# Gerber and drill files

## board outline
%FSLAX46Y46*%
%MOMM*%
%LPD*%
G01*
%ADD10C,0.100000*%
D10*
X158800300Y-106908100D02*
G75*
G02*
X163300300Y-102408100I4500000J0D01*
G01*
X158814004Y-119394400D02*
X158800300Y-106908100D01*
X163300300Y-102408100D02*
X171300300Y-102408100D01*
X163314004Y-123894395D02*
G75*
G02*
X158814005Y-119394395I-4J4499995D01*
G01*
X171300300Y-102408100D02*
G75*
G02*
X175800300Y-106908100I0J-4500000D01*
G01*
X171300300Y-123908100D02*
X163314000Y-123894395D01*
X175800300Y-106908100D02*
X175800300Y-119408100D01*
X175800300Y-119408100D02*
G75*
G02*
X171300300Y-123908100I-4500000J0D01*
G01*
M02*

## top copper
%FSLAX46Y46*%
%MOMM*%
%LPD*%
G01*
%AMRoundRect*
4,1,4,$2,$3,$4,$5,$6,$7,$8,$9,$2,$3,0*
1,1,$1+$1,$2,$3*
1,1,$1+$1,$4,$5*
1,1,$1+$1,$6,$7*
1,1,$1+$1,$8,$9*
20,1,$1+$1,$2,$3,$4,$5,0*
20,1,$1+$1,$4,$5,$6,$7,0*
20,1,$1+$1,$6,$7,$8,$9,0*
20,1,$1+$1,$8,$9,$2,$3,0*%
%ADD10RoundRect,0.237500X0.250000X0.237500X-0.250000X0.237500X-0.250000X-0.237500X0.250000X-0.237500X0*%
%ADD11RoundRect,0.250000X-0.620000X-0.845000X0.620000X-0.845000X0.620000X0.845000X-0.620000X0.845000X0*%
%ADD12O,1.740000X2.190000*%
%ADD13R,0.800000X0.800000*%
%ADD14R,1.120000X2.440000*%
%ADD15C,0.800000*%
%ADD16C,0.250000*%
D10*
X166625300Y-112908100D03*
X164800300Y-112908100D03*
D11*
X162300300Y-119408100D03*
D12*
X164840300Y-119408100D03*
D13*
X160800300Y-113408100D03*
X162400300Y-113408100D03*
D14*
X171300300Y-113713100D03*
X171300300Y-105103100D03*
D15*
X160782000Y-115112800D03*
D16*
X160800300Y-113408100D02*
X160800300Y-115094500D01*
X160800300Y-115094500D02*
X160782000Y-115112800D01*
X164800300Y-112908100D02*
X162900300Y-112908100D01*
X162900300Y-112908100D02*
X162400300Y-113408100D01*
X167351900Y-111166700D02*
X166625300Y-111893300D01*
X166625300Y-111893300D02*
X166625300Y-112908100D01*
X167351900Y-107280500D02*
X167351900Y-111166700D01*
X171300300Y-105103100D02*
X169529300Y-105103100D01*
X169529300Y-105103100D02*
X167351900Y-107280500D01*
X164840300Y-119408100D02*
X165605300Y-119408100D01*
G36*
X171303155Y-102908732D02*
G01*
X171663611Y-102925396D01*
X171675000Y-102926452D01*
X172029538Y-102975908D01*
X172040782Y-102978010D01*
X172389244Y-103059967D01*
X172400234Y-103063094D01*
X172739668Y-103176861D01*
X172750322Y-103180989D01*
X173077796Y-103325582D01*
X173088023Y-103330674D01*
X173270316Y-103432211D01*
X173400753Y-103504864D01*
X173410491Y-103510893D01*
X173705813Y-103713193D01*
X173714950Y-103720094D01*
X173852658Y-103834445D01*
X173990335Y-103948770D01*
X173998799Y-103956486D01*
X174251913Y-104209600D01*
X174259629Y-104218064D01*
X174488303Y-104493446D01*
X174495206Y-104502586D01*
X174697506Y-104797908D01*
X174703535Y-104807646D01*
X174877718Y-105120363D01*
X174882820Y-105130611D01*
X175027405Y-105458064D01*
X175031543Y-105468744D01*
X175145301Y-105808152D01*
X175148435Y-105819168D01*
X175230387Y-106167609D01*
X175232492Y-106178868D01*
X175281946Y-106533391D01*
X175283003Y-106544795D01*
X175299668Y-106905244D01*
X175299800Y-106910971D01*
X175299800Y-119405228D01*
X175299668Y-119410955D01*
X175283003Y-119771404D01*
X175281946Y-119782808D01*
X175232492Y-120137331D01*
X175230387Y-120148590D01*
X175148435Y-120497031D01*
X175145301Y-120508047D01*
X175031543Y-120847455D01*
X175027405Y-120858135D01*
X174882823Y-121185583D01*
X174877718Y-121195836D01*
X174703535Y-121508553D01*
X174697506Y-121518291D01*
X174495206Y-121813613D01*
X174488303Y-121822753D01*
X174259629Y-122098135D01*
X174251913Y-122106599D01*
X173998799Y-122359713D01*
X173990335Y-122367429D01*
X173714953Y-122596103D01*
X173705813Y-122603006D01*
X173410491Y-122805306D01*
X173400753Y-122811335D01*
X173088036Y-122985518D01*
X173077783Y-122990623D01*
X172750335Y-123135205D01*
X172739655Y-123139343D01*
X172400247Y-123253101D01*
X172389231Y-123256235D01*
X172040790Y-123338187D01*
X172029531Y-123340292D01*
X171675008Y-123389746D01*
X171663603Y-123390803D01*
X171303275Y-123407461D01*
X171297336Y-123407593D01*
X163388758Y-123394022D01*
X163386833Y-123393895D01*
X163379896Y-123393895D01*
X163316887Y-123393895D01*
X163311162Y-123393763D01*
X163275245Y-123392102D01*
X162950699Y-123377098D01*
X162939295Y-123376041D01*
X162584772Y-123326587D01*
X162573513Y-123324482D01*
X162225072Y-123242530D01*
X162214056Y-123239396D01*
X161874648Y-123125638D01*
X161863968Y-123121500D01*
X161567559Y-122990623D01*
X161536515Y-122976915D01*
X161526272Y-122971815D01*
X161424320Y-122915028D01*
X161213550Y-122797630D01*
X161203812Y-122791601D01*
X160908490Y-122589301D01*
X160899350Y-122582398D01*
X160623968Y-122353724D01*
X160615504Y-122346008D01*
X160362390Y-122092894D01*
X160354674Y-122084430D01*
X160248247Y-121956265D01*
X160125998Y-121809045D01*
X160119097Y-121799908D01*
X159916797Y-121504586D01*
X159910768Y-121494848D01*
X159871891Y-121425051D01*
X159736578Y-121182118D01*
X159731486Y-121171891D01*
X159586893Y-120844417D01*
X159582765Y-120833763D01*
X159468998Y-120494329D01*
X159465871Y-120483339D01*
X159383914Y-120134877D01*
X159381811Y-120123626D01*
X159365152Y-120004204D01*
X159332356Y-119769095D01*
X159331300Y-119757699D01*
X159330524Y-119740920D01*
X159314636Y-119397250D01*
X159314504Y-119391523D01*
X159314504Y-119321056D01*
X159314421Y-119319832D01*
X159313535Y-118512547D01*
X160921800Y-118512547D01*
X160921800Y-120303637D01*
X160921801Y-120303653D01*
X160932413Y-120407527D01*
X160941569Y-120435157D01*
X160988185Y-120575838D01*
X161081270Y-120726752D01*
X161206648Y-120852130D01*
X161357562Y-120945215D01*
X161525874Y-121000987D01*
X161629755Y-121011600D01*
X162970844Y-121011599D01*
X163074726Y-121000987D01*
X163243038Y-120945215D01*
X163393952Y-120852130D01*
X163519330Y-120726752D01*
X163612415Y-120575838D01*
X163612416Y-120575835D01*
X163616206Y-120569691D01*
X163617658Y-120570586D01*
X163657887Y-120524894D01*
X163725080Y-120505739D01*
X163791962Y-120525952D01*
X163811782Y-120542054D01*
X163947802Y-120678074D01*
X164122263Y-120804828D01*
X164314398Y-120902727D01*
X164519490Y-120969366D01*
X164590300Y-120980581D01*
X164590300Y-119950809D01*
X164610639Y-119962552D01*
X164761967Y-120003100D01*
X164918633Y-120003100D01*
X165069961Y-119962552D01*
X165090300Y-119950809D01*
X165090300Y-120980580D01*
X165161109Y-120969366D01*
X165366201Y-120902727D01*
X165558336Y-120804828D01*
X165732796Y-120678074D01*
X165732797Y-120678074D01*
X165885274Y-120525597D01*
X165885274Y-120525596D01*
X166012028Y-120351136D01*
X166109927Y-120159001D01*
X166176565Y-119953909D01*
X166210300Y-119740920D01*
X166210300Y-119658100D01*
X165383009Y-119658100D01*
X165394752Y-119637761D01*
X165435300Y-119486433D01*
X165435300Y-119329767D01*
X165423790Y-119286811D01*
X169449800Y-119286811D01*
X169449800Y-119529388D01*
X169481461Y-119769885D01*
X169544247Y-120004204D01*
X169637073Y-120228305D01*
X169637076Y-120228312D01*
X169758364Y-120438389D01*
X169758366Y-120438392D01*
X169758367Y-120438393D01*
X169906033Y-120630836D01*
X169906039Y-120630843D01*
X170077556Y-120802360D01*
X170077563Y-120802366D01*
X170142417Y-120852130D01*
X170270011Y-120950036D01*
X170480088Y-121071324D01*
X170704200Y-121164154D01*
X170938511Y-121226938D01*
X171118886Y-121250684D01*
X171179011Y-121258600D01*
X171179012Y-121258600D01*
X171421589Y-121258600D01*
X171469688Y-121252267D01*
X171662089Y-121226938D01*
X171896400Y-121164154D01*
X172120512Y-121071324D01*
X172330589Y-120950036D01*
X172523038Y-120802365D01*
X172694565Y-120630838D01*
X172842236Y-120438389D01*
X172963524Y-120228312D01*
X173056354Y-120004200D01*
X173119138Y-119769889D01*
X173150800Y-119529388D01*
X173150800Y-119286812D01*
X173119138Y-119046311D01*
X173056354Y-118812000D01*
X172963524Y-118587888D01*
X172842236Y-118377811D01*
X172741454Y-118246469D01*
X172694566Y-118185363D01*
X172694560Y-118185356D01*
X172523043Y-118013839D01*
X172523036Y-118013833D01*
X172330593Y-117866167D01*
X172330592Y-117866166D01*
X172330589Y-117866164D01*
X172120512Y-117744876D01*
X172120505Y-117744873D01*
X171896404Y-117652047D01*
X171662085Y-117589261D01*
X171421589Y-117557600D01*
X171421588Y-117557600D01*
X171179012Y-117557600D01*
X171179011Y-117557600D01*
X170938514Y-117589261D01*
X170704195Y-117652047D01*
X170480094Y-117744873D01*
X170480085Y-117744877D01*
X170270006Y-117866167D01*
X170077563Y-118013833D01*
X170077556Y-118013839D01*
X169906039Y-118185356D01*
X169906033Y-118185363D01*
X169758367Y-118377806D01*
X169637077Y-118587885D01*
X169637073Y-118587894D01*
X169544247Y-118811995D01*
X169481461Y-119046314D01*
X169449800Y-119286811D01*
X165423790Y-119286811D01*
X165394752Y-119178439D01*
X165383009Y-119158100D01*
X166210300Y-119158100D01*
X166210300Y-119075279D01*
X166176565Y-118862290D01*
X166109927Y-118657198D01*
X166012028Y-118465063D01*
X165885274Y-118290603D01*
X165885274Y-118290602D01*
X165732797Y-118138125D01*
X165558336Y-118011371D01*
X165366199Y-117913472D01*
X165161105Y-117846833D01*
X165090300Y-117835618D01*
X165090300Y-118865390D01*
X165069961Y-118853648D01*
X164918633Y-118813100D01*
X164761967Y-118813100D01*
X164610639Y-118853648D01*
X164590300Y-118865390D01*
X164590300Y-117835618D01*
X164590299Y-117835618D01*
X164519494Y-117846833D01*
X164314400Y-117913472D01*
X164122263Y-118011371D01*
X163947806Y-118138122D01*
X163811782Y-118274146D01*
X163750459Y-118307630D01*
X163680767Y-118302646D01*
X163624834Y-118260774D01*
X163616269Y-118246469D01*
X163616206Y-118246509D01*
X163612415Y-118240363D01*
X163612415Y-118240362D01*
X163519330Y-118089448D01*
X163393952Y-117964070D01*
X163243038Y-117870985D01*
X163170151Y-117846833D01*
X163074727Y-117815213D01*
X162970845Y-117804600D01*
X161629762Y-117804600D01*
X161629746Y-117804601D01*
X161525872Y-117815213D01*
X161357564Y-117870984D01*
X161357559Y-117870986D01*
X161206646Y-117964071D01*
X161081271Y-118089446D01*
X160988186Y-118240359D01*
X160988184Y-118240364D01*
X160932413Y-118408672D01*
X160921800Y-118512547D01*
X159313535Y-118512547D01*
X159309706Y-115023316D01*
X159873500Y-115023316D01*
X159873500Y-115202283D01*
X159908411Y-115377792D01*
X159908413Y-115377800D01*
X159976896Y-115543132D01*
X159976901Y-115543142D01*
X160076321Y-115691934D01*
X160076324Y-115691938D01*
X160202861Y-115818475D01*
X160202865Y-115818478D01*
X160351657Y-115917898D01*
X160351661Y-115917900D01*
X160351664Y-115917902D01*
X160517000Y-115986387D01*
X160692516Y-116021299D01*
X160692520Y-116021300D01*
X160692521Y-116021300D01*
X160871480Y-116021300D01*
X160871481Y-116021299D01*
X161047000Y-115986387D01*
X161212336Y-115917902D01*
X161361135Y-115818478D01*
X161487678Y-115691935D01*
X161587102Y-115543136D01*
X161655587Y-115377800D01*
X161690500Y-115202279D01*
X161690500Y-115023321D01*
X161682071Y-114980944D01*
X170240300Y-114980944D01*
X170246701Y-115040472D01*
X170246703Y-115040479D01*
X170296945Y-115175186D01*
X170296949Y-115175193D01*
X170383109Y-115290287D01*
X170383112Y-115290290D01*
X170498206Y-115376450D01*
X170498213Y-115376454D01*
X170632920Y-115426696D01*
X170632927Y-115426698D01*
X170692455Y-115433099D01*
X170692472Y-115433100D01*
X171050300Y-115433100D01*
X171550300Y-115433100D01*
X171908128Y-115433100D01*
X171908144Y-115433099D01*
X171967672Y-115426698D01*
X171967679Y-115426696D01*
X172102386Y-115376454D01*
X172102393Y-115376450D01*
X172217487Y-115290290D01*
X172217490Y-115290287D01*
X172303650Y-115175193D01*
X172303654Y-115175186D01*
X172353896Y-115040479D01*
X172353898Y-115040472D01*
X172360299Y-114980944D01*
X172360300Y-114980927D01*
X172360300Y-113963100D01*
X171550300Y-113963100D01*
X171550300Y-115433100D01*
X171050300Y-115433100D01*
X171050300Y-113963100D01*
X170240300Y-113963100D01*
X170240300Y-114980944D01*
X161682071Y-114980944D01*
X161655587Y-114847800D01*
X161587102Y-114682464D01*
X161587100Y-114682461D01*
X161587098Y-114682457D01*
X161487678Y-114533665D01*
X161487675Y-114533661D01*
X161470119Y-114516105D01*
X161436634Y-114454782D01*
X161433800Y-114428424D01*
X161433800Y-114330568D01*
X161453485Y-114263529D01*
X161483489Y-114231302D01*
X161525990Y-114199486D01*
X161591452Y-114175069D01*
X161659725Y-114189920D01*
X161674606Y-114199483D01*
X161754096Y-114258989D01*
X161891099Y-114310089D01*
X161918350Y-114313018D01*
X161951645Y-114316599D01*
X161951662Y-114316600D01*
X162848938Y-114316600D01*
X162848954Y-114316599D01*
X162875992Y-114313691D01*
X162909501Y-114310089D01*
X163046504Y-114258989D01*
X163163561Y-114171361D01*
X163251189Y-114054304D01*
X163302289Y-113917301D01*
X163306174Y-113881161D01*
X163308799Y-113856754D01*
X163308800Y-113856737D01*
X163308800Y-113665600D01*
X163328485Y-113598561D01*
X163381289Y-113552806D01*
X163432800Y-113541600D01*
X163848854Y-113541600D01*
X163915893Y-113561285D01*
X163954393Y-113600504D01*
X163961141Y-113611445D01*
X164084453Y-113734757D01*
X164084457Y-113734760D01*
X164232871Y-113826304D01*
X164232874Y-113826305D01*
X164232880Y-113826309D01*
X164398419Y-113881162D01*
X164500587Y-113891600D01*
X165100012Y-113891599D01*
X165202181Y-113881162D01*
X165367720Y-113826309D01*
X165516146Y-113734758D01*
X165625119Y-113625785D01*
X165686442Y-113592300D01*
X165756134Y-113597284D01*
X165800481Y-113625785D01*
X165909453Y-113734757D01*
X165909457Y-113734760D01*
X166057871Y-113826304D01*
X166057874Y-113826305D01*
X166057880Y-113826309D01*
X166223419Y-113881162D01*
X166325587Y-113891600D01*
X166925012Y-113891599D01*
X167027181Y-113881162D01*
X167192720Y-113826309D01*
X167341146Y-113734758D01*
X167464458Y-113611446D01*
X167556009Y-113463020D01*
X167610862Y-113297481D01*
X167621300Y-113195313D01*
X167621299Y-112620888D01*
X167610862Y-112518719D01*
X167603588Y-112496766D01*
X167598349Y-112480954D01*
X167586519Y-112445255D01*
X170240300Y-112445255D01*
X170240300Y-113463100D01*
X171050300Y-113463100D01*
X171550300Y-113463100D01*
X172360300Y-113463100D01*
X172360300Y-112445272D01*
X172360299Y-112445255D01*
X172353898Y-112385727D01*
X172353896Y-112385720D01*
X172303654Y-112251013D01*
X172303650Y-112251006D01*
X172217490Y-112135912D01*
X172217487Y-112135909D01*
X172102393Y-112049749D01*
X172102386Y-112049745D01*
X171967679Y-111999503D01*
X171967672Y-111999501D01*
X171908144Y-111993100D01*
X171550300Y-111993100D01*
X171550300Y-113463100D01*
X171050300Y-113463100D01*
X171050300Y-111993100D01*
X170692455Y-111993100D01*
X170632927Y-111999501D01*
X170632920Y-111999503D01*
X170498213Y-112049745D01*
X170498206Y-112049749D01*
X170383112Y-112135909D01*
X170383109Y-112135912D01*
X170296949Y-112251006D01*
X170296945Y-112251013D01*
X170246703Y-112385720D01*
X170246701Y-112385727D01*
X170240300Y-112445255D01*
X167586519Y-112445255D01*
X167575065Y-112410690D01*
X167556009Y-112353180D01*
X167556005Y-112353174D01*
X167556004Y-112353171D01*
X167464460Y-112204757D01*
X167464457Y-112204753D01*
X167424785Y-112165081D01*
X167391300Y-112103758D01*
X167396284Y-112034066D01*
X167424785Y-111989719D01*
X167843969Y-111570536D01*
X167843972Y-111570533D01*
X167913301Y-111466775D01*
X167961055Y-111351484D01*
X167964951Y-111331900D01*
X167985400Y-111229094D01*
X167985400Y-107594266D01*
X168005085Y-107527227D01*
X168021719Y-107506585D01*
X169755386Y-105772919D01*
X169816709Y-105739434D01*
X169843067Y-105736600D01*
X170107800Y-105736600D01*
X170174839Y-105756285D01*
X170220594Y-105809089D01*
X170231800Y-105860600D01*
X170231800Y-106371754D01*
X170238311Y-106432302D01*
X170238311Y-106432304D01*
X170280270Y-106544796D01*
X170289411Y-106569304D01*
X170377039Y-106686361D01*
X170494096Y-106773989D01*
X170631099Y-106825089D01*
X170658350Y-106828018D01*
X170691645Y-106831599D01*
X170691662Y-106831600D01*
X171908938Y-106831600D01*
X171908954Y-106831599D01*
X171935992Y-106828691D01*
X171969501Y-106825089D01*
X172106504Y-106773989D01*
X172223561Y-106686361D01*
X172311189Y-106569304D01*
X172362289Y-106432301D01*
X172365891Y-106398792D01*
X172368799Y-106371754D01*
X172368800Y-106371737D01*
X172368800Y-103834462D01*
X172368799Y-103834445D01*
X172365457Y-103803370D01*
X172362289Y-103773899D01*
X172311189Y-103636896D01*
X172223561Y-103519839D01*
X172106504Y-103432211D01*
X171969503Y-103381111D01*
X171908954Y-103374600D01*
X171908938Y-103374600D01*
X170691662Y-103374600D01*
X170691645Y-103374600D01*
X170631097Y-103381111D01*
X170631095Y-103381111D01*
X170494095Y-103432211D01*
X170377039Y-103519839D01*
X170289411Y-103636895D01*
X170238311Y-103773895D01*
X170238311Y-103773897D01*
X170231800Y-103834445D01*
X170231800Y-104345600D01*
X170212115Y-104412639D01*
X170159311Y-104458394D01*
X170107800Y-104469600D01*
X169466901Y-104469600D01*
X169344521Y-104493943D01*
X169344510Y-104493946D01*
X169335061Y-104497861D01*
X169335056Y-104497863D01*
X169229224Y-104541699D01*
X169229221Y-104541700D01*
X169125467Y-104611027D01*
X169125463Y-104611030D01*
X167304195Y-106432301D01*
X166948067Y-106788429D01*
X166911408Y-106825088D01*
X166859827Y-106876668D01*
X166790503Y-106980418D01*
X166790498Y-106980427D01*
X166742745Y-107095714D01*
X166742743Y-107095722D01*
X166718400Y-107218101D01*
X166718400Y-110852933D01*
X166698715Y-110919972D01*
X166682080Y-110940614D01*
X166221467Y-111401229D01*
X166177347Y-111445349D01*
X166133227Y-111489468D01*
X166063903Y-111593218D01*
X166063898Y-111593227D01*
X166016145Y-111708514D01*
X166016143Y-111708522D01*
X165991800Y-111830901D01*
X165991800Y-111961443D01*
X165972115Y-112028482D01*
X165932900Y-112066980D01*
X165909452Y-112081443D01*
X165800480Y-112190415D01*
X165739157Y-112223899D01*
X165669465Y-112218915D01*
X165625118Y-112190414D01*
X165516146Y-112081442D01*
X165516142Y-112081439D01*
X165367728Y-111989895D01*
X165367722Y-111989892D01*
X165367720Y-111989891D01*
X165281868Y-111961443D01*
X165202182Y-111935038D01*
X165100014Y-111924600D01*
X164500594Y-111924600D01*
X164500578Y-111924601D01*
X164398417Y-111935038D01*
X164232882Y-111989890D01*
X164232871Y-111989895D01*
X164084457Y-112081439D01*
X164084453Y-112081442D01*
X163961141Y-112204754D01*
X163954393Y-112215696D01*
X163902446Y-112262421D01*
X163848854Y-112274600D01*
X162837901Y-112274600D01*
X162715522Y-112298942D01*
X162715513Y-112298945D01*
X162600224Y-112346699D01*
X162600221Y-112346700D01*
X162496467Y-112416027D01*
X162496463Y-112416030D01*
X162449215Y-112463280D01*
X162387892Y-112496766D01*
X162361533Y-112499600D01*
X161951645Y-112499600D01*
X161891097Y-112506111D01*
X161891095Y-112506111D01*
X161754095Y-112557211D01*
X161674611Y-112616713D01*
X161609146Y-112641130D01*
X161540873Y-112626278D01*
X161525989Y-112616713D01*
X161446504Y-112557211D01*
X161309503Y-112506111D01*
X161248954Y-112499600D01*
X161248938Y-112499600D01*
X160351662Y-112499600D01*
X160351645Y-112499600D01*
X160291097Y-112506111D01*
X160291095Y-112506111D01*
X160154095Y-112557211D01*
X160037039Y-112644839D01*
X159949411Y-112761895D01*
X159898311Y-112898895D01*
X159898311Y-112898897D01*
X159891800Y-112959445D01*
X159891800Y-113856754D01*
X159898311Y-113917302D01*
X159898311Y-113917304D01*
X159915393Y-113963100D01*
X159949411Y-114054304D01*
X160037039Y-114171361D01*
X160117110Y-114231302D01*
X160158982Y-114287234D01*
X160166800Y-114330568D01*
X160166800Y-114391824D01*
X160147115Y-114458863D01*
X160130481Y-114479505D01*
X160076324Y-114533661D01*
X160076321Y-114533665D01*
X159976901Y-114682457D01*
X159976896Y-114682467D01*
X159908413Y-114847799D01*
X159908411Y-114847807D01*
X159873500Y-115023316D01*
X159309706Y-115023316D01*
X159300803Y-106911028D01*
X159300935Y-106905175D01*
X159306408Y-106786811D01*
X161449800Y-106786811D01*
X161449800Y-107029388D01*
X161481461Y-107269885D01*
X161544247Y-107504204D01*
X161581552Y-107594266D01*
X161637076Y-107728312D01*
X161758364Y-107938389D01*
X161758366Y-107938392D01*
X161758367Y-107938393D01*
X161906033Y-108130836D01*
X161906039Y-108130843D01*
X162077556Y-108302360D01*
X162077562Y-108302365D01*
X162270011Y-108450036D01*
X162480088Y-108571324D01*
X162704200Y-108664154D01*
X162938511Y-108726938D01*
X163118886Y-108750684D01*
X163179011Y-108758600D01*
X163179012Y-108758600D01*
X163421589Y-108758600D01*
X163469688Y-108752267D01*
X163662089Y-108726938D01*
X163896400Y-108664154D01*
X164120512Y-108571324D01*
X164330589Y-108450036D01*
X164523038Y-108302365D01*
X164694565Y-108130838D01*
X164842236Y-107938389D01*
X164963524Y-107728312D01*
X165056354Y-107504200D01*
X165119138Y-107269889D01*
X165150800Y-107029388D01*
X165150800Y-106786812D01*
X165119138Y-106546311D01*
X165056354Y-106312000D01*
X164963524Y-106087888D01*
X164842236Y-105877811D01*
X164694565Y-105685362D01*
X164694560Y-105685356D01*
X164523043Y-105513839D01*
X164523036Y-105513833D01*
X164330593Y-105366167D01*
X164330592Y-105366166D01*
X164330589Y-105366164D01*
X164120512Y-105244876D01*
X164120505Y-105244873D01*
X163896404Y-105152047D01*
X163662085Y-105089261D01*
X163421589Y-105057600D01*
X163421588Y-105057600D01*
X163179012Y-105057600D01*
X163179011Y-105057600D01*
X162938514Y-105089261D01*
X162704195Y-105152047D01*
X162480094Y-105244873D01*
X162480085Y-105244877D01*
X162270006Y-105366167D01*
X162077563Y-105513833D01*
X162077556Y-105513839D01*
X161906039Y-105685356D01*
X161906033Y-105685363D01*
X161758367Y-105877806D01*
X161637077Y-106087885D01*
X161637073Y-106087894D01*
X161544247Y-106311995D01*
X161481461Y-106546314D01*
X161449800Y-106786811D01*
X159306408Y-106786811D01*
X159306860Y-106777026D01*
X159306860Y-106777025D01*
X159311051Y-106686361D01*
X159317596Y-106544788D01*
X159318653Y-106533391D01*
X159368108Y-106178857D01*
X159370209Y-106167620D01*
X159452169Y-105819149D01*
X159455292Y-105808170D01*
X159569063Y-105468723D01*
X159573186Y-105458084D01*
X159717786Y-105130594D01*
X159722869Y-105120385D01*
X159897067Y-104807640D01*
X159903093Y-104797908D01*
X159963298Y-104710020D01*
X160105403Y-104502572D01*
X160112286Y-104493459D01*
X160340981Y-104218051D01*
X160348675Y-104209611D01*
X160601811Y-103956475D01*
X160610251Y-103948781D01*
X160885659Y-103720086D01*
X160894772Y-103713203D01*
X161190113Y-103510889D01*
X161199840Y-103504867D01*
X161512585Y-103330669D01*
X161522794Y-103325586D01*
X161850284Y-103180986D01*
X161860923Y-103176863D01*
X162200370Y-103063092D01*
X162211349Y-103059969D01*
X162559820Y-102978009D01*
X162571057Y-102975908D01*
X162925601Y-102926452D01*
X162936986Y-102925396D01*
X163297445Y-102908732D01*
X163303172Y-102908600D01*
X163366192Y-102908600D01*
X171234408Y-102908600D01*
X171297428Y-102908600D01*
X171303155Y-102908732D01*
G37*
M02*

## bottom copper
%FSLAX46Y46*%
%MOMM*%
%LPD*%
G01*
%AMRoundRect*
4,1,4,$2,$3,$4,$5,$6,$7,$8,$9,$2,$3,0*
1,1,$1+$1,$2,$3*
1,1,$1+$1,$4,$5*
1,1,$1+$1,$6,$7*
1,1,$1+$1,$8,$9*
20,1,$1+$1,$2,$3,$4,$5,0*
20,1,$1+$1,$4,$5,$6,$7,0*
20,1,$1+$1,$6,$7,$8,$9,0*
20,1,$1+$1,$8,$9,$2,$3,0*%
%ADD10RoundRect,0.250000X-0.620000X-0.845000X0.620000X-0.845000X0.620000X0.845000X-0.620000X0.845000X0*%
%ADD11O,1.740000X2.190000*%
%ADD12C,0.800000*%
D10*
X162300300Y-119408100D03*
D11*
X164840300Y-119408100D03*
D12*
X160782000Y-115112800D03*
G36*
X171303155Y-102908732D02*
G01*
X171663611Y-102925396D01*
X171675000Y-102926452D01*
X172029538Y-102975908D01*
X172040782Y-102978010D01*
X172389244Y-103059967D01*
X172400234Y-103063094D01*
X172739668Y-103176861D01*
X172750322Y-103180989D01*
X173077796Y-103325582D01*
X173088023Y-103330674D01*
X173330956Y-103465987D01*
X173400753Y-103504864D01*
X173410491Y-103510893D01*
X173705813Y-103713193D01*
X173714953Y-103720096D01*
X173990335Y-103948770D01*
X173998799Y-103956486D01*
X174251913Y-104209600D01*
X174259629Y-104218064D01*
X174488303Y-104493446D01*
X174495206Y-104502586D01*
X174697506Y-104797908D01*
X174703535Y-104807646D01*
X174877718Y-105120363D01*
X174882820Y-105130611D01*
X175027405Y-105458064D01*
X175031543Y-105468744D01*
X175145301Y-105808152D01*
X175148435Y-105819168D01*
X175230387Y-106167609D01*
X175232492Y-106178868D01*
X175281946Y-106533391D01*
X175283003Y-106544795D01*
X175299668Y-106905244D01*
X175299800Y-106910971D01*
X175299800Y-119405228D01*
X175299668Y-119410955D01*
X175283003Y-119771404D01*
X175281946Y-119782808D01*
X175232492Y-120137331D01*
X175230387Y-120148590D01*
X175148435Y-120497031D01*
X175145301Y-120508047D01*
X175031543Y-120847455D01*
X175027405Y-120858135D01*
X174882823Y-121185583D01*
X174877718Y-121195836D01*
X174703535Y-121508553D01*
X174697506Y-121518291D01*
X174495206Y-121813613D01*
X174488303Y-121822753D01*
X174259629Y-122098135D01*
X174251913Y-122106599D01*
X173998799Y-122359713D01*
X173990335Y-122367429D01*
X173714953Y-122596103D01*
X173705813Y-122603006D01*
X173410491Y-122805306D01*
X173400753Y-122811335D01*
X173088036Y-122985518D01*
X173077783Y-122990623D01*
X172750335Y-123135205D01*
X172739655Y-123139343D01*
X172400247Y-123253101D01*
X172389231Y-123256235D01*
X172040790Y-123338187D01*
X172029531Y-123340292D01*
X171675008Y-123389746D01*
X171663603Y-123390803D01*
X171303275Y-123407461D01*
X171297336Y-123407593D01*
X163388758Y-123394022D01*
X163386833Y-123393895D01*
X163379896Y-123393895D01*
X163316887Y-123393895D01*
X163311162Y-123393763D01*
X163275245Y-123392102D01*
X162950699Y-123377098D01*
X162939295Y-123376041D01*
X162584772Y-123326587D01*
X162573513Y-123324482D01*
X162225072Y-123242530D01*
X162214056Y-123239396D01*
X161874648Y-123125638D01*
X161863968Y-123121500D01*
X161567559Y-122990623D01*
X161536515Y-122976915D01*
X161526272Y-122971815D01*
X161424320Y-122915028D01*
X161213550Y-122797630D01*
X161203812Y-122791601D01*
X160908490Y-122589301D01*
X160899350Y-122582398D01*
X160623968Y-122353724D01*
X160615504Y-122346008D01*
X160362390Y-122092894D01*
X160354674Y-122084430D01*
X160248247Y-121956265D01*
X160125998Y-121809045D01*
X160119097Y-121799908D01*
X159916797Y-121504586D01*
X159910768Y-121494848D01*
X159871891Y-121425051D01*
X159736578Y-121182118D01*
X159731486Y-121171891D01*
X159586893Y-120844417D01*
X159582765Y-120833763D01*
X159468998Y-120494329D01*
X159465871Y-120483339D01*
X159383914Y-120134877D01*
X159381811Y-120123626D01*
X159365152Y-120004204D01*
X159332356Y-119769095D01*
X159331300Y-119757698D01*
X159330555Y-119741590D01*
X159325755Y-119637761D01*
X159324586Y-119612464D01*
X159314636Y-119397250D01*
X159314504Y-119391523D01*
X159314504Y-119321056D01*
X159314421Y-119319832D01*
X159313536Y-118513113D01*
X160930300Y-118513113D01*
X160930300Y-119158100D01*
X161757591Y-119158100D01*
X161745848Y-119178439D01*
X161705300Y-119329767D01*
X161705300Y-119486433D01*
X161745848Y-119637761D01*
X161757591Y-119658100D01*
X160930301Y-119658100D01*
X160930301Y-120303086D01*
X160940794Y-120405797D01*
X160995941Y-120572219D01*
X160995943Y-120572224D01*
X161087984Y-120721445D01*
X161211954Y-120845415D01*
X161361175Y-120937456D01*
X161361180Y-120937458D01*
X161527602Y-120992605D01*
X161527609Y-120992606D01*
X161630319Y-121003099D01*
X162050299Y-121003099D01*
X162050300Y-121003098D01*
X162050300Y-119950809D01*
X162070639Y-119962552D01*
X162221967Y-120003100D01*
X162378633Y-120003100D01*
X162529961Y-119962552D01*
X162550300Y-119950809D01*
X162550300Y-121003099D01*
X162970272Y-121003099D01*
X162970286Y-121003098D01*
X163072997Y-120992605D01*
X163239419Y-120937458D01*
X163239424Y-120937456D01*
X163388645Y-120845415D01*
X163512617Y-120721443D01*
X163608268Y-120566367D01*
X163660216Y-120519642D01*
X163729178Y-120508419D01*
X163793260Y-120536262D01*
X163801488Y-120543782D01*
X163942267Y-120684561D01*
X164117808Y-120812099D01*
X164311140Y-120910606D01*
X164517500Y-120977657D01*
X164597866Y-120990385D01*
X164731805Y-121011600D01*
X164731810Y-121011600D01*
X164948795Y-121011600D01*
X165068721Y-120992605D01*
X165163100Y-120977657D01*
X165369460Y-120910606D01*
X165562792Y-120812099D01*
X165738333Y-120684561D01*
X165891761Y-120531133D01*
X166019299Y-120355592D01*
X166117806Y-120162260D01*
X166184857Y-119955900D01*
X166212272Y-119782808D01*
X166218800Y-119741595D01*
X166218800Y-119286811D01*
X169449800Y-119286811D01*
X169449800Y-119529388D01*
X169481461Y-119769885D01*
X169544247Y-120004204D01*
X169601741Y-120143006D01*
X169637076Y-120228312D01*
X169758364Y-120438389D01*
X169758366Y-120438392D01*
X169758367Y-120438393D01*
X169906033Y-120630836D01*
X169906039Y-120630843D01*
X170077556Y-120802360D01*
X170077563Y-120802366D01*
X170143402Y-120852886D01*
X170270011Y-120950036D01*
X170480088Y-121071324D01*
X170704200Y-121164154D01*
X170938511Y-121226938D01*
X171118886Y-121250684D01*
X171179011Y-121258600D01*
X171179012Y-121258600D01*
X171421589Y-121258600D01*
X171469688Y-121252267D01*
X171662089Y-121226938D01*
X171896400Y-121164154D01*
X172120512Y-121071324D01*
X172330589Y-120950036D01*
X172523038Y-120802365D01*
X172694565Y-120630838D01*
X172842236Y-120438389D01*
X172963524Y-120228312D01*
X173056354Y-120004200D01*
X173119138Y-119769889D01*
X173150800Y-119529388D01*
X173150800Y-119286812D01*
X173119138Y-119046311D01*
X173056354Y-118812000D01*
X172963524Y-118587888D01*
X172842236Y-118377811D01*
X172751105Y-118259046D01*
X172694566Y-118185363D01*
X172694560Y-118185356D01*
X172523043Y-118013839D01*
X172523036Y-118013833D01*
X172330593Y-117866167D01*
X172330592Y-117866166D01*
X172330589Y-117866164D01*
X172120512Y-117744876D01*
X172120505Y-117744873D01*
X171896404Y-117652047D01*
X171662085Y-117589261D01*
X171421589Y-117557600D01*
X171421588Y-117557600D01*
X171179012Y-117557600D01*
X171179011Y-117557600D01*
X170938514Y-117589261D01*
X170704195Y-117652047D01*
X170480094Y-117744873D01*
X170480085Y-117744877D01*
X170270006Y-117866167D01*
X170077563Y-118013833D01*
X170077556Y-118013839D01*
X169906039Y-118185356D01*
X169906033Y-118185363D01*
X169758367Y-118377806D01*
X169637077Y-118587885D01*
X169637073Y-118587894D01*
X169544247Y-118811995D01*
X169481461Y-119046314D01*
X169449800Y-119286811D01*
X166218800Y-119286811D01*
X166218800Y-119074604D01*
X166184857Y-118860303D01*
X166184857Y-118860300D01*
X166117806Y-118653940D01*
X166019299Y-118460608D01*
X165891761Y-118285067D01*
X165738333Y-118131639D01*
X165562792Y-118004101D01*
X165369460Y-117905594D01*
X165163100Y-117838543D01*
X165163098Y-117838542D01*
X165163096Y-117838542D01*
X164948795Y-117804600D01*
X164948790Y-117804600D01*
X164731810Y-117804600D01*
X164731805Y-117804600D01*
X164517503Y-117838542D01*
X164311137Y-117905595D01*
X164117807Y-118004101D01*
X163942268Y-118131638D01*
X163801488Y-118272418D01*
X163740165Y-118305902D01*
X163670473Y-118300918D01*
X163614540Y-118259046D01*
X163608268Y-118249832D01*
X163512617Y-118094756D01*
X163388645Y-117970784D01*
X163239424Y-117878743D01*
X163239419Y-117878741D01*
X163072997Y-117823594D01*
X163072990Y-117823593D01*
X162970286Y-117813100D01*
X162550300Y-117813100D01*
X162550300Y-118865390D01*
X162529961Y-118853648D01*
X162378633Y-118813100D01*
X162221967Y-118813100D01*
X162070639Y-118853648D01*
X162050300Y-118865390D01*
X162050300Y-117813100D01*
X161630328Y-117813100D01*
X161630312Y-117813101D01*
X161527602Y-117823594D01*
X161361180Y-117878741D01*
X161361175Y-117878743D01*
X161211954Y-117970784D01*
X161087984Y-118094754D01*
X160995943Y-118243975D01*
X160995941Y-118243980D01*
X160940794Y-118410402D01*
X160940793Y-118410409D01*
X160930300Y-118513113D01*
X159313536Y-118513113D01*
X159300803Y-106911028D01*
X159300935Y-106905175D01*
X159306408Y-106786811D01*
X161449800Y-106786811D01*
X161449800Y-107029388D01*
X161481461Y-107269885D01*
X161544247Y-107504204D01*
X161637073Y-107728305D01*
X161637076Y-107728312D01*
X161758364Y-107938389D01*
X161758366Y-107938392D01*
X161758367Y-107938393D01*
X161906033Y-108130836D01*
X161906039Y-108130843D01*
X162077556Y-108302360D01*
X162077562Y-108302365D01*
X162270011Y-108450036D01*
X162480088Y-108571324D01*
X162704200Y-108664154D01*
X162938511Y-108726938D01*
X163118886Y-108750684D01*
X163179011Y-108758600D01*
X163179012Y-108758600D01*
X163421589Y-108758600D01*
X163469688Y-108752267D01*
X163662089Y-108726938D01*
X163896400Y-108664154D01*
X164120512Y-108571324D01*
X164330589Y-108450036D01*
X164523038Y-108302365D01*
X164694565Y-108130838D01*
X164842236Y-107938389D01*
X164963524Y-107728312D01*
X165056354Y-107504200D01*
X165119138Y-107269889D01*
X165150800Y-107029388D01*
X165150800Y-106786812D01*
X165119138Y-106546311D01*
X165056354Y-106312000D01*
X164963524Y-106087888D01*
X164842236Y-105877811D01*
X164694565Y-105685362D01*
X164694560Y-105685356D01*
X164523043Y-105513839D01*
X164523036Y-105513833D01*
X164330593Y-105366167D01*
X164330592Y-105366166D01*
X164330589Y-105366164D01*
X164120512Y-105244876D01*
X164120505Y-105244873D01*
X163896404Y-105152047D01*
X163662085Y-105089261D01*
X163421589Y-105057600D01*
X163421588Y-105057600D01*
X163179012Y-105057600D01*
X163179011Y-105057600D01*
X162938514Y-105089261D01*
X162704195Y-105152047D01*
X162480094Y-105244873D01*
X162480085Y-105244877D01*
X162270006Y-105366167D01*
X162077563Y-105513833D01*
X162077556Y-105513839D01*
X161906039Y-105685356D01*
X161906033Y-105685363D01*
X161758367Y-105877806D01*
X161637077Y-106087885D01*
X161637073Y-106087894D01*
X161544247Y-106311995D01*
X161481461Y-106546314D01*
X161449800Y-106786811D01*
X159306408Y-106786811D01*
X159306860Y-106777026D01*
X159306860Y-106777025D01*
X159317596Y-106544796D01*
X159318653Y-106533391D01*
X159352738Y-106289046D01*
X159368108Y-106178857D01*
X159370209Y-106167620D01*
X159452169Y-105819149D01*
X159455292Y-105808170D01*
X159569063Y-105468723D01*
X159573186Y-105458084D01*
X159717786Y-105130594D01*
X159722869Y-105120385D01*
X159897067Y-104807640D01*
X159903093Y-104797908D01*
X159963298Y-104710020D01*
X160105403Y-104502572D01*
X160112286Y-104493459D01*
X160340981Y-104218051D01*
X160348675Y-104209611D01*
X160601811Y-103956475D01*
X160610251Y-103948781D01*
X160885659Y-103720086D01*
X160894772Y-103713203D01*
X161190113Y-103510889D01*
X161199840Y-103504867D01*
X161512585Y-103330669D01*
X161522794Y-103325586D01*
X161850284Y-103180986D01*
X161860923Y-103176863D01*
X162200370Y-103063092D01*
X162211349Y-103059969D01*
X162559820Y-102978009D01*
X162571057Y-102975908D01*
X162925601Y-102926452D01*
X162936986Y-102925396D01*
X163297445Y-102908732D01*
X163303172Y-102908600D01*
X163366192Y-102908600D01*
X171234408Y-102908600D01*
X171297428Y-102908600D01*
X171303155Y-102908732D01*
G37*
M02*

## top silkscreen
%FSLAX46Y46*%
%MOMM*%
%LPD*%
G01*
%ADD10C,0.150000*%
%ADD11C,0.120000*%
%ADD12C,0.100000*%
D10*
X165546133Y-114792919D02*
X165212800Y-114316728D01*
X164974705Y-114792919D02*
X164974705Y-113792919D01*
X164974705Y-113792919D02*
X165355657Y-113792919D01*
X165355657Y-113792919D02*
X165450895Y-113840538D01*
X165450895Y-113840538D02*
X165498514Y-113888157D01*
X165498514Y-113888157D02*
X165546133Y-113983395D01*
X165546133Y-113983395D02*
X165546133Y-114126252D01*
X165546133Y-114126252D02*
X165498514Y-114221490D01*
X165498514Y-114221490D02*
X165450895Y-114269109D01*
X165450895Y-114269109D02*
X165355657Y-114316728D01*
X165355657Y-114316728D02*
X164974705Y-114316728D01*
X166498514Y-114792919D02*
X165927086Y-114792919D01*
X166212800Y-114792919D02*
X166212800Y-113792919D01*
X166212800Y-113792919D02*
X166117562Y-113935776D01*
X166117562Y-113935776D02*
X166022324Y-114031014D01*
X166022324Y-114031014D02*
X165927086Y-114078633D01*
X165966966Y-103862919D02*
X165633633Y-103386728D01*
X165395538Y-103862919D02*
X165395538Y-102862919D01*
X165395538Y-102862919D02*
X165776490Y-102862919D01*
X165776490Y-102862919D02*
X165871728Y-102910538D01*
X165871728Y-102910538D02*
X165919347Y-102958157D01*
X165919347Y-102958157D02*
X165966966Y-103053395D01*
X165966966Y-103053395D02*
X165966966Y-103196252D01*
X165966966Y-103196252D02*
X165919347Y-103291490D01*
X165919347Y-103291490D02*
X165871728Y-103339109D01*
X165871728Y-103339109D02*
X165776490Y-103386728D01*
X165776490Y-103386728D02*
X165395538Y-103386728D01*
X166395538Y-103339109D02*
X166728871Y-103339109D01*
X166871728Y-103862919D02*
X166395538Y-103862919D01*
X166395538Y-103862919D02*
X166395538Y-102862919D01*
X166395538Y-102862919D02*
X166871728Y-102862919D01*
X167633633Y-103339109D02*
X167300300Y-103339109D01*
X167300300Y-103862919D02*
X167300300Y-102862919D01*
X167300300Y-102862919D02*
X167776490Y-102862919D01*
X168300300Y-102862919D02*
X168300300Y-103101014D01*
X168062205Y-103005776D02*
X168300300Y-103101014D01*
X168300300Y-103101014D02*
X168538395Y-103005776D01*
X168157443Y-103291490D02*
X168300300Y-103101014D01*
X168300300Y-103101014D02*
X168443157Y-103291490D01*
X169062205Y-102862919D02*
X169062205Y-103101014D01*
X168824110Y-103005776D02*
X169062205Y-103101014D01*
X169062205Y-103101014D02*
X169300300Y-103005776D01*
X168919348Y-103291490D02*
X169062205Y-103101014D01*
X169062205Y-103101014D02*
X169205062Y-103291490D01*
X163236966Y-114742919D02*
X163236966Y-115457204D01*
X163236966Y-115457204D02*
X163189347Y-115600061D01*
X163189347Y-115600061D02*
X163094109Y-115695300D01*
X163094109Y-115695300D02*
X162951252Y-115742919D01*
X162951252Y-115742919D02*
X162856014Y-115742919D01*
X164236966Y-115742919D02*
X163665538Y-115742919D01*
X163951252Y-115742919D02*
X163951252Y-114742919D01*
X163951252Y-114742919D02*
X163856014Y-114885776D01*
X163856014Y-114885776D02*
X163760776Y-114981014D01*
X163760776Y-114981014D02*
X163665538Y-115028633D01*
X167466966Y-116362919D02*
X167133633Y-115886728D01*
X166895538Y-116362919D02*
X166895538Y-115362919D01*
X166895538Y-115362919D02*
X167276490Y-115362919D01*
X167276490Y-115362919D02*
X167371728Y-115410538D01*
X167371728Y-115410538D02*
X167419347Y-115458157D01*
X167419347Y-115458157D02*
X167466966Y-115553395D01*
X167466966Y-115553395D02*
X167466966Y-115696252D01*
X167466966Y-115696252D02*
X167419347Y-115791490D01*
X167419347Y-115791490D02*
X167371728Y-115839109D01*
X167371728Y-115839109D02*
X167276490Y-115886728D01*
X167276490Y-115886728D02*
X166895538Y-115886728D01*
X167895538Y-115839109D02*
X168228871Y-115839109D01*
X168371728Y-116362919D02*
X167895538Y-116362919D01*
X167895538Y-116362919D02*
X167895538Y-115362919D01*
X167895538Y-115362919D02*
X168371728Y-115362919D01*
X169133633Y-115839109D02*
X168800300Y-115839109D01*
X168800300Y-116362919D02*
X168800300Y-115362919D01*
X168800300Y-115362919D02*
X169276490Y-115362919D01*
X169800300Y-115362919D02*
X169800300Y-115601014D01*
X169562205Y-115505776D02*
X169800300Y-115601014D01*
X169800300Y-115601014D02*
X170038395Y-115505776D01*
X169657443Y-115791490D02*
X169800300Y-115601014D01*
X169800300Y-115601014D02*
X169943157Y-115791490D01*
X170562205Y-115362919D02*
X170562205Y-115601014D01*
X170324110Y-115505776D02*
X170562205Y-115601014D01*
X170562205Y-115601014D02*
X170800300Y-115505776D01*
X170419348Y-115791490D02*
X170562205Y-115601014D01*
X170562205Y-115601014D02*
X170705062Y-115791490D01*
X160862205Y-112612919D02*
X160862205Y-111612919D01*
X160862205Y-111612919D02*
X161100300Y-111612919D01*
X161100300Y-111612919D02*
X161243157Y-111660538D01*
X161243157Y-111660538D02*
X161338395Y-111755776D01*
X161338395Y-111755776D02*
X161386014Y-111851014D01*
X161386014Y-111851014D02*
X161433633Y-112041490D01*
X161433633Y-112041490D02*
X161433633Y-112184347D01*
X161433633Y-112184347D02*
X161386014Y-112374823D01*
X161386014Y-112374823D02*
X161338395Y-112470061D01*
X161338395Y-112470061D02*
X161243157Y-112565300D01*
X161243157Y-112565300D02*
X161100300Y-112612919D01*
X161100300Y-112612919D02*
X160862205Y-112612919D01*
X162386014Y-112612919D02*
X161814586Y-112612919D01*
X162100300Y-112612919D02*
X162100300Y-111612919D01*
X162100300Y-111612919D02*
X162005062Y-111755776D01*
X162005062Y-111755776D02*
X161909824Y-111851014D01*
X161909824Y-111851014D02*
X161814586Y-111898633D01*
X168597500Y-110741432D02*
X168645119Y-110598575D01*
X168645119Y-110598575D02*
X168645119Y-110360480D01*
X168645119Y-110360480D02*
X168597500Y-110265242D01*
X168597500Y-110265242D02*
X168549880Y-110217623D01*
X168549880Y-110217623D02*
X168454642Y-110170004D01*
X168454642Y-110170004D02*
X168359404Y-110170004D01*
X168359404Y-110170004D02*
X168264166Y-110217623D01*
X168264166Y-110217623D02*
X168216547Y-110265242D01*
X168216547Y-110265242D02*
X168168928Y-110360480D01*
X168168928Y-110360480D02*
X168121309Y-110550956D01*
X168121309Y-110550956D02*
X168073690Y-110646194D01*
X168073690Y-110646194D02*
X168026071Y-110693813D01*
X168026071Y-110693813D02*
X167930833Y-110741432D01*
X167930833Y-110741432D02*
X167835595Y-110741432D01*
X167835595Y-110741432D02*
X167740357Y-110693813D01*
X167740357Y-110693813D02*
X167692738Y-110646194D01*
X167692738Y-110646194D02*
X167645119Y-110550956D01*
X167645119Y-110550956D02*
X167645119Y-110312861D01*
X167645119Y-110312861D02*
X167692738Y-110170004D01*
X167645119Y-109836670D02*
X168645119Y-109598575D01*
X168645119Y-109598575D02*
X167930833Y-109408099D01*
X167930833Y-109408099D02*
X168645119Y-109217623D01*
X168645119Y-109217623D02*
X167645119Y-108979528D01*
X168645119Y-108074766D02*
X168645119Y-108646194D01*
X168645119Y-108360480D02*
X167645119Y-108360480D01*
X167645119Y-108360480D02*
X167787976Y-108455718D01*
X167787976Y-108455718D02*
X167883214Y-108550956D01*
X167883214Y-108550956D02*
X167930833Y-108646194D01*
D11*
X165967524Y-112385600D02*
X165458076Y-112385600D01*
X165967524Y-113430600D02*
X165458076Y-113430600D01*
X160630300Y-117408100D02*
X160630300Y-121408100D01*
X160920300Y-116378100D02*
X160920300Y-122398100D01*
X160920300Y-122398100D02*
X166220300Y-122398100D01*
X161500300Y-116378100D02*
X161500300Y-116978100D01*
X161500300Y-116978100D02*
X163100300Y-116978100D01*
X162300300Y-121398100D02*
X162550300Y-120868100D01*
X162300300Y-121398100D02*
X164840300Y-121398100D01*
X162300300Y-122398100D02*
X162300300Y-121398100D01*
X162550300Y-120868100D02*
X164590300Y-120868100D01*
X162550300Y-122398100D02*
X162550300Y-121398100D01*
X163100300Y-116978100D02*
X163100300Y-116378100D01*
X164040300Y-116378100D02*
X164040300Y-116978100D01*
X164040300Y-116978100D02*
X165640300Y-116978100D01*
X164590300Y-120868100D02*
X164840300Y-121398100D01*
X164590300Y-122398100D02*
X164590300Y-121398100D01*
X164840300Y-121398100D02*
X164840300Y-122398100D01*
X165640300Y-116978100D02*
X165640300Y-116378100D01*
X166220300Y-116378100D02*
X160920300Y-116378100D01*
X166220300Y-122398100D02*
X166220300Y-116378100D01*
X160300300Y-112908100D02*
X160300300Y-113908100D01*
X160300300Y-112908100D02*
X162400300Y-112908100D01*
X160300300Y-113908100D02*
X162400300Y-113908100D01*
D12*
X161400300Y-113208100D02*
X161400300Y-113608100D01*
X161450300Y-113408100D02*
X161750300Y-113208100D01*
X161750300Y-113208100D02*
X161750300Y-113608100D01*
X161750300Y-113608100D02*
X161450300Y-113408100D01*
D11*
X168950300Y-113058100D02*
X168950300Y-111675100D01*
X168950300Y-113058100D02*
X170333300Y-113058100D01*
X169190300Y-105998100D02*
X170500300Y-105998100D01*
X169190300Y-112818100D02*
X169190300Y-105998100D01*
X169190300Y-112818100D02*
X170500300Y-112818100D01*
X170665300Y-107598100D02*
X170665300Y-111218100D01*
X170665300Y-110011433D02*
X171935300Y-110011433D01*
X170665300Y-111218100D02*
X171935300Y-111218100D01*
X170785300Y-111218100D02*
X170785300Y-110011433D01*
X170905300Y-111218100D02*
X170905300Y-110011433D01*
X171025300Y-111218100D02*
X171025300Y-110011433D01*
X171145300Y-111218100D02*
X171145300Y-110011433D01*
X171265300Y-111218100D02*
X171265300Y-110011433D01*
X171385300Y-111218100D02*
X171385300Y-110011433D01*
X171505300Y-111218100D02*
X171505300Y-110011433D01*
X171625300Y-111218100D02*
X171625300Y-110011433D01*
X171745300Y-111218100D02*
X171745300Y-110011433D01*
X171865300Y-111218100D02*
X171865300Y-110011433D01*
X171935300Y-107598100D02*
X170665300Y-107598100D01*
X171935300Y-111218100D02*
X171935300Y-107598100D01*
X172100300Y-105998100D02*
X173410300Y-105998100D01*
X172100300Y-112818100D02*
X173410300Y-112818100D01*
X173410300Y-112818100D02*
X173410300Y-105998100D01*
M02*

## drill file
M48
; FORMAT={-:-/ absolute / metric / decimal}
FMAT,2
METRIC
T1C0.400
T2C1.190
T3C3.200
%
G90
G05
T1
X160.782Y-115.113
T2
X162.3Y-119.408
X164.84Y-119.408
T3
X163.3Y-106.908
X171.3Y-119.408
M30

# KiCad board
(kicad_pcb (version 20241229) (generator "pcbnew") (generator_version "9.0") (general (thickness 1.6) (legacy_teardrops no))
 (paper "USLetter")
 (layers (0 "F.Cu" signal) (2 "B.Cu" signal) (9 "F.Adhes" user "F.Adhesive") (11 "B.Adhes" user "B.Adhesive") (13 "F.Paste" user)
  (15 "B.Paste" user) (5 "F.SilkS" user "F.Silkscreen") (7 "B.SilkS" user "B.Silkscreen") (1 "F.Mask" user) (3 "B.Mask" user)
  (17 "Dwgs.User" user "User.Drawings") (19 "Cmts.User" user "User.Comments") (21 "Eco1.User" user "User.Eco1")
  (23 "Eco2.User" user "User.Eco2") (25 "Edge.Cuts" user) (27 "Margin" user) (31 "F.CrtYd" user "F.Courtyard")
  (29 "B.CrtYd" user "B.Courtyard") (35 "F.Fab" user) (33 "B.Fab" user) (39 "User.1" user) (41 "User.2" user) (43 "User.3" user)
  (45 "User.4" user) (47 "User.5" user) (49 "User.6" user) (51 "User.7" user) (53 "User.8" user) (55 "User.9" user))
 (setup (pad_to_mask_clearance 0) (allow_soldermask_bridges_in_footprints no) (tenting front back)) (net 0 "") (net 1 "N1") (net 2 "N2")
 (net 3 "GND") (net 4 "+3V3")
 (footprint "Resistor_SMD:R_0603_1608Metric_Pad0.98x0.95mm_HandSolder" (layer "F.Cu") (at 165.7128 112.9081 180)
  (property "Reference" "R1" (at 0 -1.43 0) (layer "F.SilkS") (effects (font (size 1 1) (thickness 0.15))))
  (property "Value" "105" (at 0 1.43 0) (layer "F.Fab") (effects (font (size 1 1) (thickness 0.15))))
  (fp_line (start -0.254724 0.5225) (end 0.254724 0.5225) (stroke (width 0.12) (type solid)) (layer "F.SilkS"))
  (fp_line (start -0.254724 -0.5225) (end 0.254724 -0.5225) (stroke (width 0.12) (type solid)) (layer "F.SilkS"))
  (pad "1" smd roundrect (at -0.9125 0 180) (size 0.975 0.95) (layers "F.Cu" "F.Mask" "F.Paste") (roundrect_rratio 0.25) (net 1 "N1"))
  (pad "2" smd roundrect (at 0.9125 0 180) (size 0.975 0.95) (layers "F.Cu" "F.Mask" "F.Paste") (roundrect_rratio 0.25) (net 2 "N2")))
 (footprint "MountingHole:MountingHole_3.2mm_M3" (layer "F.Cu") (at 163.3003 106.9081)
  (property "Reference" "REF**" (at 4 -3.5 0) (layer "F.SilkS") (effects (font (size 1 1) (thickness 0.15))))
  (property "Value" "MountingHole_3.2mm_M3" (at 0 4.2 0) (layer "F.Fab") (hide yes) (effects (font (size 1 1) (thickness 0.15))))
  (pad "" np_thru_hole circle (at 0 0) (size 3.2 3.2) (drill 3.2) (layers "*.Cu" "*.Mask")))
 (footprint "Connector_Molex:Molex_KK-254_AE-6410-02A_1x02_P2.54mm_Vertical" (layer "F.Cu") (at 162.3003 119.4081)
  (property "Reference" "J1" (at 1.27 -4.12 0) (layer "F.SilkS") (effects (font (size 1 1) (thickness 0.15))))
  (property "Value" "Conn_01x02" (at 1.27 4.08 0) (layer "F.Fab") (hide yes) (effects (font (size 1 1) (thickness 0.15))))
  (fp_line (start -1.67 -2) (end -1.67 2) (stroke (width 0.12) (type solid)) (layer "F.SilkS"))
  (fp_line (start -1.38 -3.03) (end -1.38 2.99) (stroke (width 0.12) (type solid)) (layer "F.SilkS"))
  (fp_line (start -1.38 2.99) (end 3.92 2.99) (stroke (width 0.12) (type solid)) (layer "F.SilkS"))
  (fp_line (start -0.8 -3.03) (end -0.8 -2.43) (stroke (width 0.12) (type solid)) (layer "F.SilkS"))
  (fp_line (start -0.8 -2.43) (end 0.8 -2.43) (stroke (width 0.12) (type solid)) (layer "F.SilkS"))
  (fp_line (start 0 1.99) (end 0.25 1.46) (stroke (width 0.12) (type solid)) (layer "F.SilkS"))
  (fp_line (start 0 1.99) (end 2.54 1.99) (stroke (width 0.12) (type solid)) (layer "F.SilkS"))
  (fp_line (start 0 2.99) (end 0 1.99) (stroke (width 0.12) (type solid)) (layer "F.SilkS"))
  (fp_line (start 0.25 1.46) (end 2.29 1.46) (stroke (width 0.12) (type solid)) (layer "F.SilkS"))
  (fp_line (start 0.25 2.99) (end 0.25 1.99) (stroke (width 0.12) (type solid)) (layer "F.SilkS"))
  (fp_line (start 0.8 -2.43) (end 0.8 -3.03) (stroke (width 0.12) (type solid)) (layer "F.SilkS"))
  (fp_line (start 1.74 -3.03) (end 1.74 -2.43) (stroke (width 0.12) (type solid)) (layer "F.SilkS"))
  (fp_line (start 1.74 -2.43) (end 3.34 -2.43) (stroke (width 0.12) (type solid)) (layer "F.SilkS"))
  (fp_line (start 2.29 1.46) (end 2.54 1.99) (stroke (width 0.12) (type solid)) (layer "F.SilkS"))
  (fp_line (start 2.29 2.99) (end 2.29 1.99) (stroke (width 0.12) (type solid)) (layer "F.SilkS"))
  (fp_line (start 2.54 1.99) (end 2.54 2.99) (stroke (width 0.12) (type solid)) (layer "F.SilkS"))
  (fp_line (start 3.34 -2.43) (end 3.34 -3.03) (stroke (width 0.12) (type solid)) (layer "F.SilkS"))
  (fp_line (start 3.92 -3.03) (end -1.38 -3.03) (stroke (width 0.12) (type solid)) (layer "F.SilkS"))
  (fp_line (start 3.92 2.99) (end 3.92 -3.03) (stroke (width 0.12) (type solid)) (layer "F.SilkS"))
  (pad "1" thru_hole roundrect (at 0 0) (size 1.74 2.19) (drill 1.19) (layers "*.Cu" "*.Mask") (remove_unused_layers no)
   (roundrect_rratio 0.143678) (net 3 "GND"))
  (pad "2" thru_hole oval (at 2.54 0) (size 1.74 2.19) (drill 1.19) (layers "*.Cu" "*.Mask") (remove_unused_layers no) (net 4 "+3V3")))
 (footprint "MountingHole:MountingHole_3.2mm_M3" (layer "F.Cu") (at 171.3003 119.4081)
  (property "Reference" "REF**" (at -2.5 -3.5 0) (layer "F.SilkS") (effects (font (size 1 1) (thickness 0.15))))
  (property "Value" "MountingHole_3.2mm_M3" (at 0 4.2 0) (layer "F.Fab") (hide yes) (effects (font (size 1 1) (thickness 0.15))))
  (pad "" np_thru_hole circle (at 0 0) (size 3.2 3.2) (drill 3.2) (layers "*.Cu" "*.Mask")))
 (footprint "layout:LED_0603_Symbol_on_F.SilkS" (layer "F.Cu") (at 161.6003 113.4081)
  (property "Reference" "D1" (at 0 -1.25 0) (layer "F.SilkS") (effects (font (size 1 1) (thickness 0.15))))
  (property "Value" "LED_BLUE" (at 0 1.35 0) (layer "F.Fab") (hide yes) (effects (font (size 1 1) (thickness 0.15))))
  (fp_line (start -1.3 -0.5) (end -1.3 0.5) (stroke (width 0.12) (type solid)) (layer "F.SilkS"))
  (fp_line (start -1.3 -0.5) (end 0.8 -0.5) (stroke (width 0.12) (type solid)) (layer "F.SilkS"))
  (fp_line (start -1.3 0.5) (end 0.8 0.5) (stroke (width 0.12) (type solid)) (layer "F.SilkS"))
  (fp_line (start -0.2 -0.2) (end -0.2 0.2) (stroke (width 0.1) (type solid)) (layer "F.SilkS"))
  (fp_line (start -0.15 0) (end 0.15 -0.2) (stroke (width 0.1) (type solid)) (layer "F.SilkS"))
  (fp_line (start 0.15 -0.2) (end 0.15 0.2) (stroke (width 0.1) (type solid)) (layer "F.SilkS"))
  (fp_line (start 0.15 0.2) (end -0.15 0) (stroke (width 0.1) (type solid)) (layer "F.SilkS"))
  (pad "1" smd rect (at -0.8 0 180) (size 0.8 0.8) (layers "F.Cu" "F.Mask" "F.Paste") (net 3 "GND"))
  (pad "2" smd rect (at 0.8 0 180) (size 0.8 0.8) (layers "F.Cu" "F.Mask" "F.Paste") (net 2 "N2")))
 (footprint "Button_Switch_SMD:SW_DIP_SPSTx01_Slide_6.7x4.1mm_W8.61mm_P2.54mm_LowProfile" (layer "F.Cu") (at 171.3003 109.4081 90)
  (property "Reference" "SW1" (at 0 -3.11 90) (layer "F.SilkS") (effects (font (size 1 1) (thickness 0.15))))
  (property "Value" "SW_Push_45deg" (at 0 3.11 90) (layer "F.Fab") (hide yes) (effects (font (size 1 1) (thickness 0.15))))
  (fp_line (start -3.65 -2.35) (end -2.267 -2.35) (stroke (width 0.12) (type solid)) (layer "F.SilkS"))
  (fp_line (start -3.65 -2.35) (end -3.65 -0.967) (stroke (width 0.12) (type solid)) (layer "F.SilkS"))
  (fp_line (start 3.41 -2.11) (end 3.41 -0.8) (stroke (width 0.12) (type solid)) (layer "F.SilkS"))
  (fp_line (start -3.41 -2.11) (end 3.41 -2.11) (stroke (width 0.12) (type solid)) (layer "F.SilkS"))
  (fp_line (start -3.41 -2.11) (end -3.41 -0.8) (stroke (width 0.12) (type solid)) (layer "F.SilkS"))
  (fp_line (start 1.81 -0.635) (end -1.81 -0.635) (stroke (width 0.12) (type solid)) (layer "F.SilkS"))
  (fp_line (start -0.603333 -0.635) (end -0.603333 0.635) (stroke (width 0.12) (type solid)) (layer "F.SilkS"))
  (fp_line (start -1.81 -0.635) (end -1.81 0.635) (stroke (width 0.12) (type solid)) (layer "F.SilkS"))
  (fp_line (start -1.81 -0.515) (end -0.603333 -0.515) (stroke (width 0.12) (type solid)) (layer "F.SilkS"))
  (fp_line (start -1.81 -0.395) (end -0.603333 -0.395) (stroke (width 0.12) (type solid)) (layer "F.SilkS"))
  (fp_line (start -1.81 -0.275) (end -0.603333 -0.275) (stroke (width 0.12) (type solid)) (layer "F.SilkS"))
  (fp_line (start -1.81 -0.155) (end -0.603333 -0.155) (stroke (width 0.12) (type solid)) (layer "F.SilkS"))
  (fp_line (start -1.81 -0.035) (end -0.603333 -0.035) (stroke (width 0.12) (type solid)) (layer "F.SilkS"))
  (fp_line (start -1.81 0.085) (end -0.603333 0.085) (stroke (width 0.12) (type solid)) (layer "F.SilkS"))
  (fp_line (start -1.81 0.205) (end -0.603333 0.205) (stroke (width 0.12) (type solid)) (layer "F.SilkS"))
  (fp_line (start -1.81 0.325) (end -0.603333 0.325) (stroke (width 0.12) (type solid)) (layer "F.SilkS"))
  (fp_line (start -1.81 0.445) (end -0.603333 0.445) (stroke (width 0.12) (type solid)) (layer "F.SilkS"))
  (fp_line (start -1.81 0.565) (end -0.603333 0.565) (stroke (width 0.12) (type solid)) (layer "F.SilkS"))
  (fp_line (start 1.81 0.635) (end 1.81 -0.635) (stroke (width 0.12) (type solid)) (layer "F.SilkS"))
  (fp_line (start -1.81 0.635) (end 1.81 0.635) (stroke (width 0.12) (type solid)) (layer "F.SilkS"))
  (fp_line (start 3.41 0.8) (end 3.41 2.11) (stroke (width 0.12) (type solid)) (layer "F.SilkS"))
  (fp_line (start -3.41 0.8) (end -3.41 2.11) (stroke (width 0.12) (type solid)) (layer "F.SilkS"))
  (fp_line (start -3.41 2.11) (end 3.41 2.11) (stroke (width 0.12) (type solid)) (layer "F.SilkS"))
  (pad "1" smd rect (at -4.305 0 90) (size 2.44 1.12) (layers "F.Cu" "F.Mask" "F.Paste") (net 4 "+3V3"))
  (pad "2" smd rect (at 4.305 0 90) (size 2.44 1.12) (layers "F.Cu" "F.Mask" "F.Paste") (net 1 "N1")))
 (gr_arc (start 158.8003 106.9081) (mid 160.118319 103.726119) (end 163.3003 102.4081) (stroke (width 0.1) (type default))
  (layer "Edge.Cuts"))
 (gr_line (start 158.814004 119.3944) (end 158.8003 106.9081) (stroke (width 0.1) (type default)) (layer "Edge.Cuts"))
 (gr_line (start 163.3003 102.4081) (end 171.3003 102.4081) (stroke (width 0.1) (type default)) (layer "Edge.Cuts"))
 (gr_arc (start 163.314004 123.894395) (mid 160.132023 122.576376) (end 158.814004 119.394395) (stroke (width 0.1) (type default))
  (layer "Edge.Cuts"))
 (gr_arc (start 171.3003 102.4081) (mid 174.482281 103.726119) (end 175.8003 106.9081) (stroke (width 0.1) (type default))
  (layer "Edge.Cuts"))
 (gr_line (start 171.3003 123.9081) (end 163.314 123.894395) (stroke (width 0.1) (type default)) (layer "Edge.Cuts"))
 (gr_line (start 175.8003 106.9081) (end 175.8003 119.4081) (stroke (width 0.1) (type default)) (layer "Edge.Cuts"))
 (gr_arc (start 175.8003 119.4081) (mid 174.482281 122.590081) (end 171.3003 123.9081) (stroke (width 0.1) (type default))
  (layer "Edge.Cuts"))
 (segment (start 160.8003 113.4081) (end 160.8003 115.0945) (width 0.25) (layer "F.Cu") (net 3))
 (segment (start 160.8003 115.0945) (end 160.782 115.1128) (width 0.25) (layer "F.Cu") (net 3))
 (via (at 160.782 115.1128) (size 0.8) (drill 0.4) (layers "F.Cu" "B.Cu") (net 3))
 (segment (start 164.8003 112.9081) (end 162.9003 112.9081) (width 0.25) (layer "F.Cu") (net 2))
 (segment (start 162.9003 112.9081) (end 162.4003 113.4081) (width 0.25) (layer "F.Cu") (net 2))
 (segment (start 167.3519 111.1667) (end 166.6253 111.8933) (width 0.25) (layer "F.Cu") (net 1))
 (segment (start 166.6253 111.8933) (end 166.6253 112.9081) (width 0.25) (layer "F.Cu") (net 1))
 (segment (start 167.3519 107.2805) (end 167.3519 111.1667) (width 0.25) (layer "F.Cu") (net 1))
 (segment (start 171.3003 105.1031) (end 169.5293 105.1031) (width 0.25) (layer "F.Cu") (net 1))
 (segment (start 169.5293 105.1031) (end 167.3519 107.2805) (width 0.25) (layer "F.Cu") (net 1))
 (segment (start 164.8403 119.4081) (end 165.6053 119.4081) (width 0.25) (layer "F.Cu") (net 4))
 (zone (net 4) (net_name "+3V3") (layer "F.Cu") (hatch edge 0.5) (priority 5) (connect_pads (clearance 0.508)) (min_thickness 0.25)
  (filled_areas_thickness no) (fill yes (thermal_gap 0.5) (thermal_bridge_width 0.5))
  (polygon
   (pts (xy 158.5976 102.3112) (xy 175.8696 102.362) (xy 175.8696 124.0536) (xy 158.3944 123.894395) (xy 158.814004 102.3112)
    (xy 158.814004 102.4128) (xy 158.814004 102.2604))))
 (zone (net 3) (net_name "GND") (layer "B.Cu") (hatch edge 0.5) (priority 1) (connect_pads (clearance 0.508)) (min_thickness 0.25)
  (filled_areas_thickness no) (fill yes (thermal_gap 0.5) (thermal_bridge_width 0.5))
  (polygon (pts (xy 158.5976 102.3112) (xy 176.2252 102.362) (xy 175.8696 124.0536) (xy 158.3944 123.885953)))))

